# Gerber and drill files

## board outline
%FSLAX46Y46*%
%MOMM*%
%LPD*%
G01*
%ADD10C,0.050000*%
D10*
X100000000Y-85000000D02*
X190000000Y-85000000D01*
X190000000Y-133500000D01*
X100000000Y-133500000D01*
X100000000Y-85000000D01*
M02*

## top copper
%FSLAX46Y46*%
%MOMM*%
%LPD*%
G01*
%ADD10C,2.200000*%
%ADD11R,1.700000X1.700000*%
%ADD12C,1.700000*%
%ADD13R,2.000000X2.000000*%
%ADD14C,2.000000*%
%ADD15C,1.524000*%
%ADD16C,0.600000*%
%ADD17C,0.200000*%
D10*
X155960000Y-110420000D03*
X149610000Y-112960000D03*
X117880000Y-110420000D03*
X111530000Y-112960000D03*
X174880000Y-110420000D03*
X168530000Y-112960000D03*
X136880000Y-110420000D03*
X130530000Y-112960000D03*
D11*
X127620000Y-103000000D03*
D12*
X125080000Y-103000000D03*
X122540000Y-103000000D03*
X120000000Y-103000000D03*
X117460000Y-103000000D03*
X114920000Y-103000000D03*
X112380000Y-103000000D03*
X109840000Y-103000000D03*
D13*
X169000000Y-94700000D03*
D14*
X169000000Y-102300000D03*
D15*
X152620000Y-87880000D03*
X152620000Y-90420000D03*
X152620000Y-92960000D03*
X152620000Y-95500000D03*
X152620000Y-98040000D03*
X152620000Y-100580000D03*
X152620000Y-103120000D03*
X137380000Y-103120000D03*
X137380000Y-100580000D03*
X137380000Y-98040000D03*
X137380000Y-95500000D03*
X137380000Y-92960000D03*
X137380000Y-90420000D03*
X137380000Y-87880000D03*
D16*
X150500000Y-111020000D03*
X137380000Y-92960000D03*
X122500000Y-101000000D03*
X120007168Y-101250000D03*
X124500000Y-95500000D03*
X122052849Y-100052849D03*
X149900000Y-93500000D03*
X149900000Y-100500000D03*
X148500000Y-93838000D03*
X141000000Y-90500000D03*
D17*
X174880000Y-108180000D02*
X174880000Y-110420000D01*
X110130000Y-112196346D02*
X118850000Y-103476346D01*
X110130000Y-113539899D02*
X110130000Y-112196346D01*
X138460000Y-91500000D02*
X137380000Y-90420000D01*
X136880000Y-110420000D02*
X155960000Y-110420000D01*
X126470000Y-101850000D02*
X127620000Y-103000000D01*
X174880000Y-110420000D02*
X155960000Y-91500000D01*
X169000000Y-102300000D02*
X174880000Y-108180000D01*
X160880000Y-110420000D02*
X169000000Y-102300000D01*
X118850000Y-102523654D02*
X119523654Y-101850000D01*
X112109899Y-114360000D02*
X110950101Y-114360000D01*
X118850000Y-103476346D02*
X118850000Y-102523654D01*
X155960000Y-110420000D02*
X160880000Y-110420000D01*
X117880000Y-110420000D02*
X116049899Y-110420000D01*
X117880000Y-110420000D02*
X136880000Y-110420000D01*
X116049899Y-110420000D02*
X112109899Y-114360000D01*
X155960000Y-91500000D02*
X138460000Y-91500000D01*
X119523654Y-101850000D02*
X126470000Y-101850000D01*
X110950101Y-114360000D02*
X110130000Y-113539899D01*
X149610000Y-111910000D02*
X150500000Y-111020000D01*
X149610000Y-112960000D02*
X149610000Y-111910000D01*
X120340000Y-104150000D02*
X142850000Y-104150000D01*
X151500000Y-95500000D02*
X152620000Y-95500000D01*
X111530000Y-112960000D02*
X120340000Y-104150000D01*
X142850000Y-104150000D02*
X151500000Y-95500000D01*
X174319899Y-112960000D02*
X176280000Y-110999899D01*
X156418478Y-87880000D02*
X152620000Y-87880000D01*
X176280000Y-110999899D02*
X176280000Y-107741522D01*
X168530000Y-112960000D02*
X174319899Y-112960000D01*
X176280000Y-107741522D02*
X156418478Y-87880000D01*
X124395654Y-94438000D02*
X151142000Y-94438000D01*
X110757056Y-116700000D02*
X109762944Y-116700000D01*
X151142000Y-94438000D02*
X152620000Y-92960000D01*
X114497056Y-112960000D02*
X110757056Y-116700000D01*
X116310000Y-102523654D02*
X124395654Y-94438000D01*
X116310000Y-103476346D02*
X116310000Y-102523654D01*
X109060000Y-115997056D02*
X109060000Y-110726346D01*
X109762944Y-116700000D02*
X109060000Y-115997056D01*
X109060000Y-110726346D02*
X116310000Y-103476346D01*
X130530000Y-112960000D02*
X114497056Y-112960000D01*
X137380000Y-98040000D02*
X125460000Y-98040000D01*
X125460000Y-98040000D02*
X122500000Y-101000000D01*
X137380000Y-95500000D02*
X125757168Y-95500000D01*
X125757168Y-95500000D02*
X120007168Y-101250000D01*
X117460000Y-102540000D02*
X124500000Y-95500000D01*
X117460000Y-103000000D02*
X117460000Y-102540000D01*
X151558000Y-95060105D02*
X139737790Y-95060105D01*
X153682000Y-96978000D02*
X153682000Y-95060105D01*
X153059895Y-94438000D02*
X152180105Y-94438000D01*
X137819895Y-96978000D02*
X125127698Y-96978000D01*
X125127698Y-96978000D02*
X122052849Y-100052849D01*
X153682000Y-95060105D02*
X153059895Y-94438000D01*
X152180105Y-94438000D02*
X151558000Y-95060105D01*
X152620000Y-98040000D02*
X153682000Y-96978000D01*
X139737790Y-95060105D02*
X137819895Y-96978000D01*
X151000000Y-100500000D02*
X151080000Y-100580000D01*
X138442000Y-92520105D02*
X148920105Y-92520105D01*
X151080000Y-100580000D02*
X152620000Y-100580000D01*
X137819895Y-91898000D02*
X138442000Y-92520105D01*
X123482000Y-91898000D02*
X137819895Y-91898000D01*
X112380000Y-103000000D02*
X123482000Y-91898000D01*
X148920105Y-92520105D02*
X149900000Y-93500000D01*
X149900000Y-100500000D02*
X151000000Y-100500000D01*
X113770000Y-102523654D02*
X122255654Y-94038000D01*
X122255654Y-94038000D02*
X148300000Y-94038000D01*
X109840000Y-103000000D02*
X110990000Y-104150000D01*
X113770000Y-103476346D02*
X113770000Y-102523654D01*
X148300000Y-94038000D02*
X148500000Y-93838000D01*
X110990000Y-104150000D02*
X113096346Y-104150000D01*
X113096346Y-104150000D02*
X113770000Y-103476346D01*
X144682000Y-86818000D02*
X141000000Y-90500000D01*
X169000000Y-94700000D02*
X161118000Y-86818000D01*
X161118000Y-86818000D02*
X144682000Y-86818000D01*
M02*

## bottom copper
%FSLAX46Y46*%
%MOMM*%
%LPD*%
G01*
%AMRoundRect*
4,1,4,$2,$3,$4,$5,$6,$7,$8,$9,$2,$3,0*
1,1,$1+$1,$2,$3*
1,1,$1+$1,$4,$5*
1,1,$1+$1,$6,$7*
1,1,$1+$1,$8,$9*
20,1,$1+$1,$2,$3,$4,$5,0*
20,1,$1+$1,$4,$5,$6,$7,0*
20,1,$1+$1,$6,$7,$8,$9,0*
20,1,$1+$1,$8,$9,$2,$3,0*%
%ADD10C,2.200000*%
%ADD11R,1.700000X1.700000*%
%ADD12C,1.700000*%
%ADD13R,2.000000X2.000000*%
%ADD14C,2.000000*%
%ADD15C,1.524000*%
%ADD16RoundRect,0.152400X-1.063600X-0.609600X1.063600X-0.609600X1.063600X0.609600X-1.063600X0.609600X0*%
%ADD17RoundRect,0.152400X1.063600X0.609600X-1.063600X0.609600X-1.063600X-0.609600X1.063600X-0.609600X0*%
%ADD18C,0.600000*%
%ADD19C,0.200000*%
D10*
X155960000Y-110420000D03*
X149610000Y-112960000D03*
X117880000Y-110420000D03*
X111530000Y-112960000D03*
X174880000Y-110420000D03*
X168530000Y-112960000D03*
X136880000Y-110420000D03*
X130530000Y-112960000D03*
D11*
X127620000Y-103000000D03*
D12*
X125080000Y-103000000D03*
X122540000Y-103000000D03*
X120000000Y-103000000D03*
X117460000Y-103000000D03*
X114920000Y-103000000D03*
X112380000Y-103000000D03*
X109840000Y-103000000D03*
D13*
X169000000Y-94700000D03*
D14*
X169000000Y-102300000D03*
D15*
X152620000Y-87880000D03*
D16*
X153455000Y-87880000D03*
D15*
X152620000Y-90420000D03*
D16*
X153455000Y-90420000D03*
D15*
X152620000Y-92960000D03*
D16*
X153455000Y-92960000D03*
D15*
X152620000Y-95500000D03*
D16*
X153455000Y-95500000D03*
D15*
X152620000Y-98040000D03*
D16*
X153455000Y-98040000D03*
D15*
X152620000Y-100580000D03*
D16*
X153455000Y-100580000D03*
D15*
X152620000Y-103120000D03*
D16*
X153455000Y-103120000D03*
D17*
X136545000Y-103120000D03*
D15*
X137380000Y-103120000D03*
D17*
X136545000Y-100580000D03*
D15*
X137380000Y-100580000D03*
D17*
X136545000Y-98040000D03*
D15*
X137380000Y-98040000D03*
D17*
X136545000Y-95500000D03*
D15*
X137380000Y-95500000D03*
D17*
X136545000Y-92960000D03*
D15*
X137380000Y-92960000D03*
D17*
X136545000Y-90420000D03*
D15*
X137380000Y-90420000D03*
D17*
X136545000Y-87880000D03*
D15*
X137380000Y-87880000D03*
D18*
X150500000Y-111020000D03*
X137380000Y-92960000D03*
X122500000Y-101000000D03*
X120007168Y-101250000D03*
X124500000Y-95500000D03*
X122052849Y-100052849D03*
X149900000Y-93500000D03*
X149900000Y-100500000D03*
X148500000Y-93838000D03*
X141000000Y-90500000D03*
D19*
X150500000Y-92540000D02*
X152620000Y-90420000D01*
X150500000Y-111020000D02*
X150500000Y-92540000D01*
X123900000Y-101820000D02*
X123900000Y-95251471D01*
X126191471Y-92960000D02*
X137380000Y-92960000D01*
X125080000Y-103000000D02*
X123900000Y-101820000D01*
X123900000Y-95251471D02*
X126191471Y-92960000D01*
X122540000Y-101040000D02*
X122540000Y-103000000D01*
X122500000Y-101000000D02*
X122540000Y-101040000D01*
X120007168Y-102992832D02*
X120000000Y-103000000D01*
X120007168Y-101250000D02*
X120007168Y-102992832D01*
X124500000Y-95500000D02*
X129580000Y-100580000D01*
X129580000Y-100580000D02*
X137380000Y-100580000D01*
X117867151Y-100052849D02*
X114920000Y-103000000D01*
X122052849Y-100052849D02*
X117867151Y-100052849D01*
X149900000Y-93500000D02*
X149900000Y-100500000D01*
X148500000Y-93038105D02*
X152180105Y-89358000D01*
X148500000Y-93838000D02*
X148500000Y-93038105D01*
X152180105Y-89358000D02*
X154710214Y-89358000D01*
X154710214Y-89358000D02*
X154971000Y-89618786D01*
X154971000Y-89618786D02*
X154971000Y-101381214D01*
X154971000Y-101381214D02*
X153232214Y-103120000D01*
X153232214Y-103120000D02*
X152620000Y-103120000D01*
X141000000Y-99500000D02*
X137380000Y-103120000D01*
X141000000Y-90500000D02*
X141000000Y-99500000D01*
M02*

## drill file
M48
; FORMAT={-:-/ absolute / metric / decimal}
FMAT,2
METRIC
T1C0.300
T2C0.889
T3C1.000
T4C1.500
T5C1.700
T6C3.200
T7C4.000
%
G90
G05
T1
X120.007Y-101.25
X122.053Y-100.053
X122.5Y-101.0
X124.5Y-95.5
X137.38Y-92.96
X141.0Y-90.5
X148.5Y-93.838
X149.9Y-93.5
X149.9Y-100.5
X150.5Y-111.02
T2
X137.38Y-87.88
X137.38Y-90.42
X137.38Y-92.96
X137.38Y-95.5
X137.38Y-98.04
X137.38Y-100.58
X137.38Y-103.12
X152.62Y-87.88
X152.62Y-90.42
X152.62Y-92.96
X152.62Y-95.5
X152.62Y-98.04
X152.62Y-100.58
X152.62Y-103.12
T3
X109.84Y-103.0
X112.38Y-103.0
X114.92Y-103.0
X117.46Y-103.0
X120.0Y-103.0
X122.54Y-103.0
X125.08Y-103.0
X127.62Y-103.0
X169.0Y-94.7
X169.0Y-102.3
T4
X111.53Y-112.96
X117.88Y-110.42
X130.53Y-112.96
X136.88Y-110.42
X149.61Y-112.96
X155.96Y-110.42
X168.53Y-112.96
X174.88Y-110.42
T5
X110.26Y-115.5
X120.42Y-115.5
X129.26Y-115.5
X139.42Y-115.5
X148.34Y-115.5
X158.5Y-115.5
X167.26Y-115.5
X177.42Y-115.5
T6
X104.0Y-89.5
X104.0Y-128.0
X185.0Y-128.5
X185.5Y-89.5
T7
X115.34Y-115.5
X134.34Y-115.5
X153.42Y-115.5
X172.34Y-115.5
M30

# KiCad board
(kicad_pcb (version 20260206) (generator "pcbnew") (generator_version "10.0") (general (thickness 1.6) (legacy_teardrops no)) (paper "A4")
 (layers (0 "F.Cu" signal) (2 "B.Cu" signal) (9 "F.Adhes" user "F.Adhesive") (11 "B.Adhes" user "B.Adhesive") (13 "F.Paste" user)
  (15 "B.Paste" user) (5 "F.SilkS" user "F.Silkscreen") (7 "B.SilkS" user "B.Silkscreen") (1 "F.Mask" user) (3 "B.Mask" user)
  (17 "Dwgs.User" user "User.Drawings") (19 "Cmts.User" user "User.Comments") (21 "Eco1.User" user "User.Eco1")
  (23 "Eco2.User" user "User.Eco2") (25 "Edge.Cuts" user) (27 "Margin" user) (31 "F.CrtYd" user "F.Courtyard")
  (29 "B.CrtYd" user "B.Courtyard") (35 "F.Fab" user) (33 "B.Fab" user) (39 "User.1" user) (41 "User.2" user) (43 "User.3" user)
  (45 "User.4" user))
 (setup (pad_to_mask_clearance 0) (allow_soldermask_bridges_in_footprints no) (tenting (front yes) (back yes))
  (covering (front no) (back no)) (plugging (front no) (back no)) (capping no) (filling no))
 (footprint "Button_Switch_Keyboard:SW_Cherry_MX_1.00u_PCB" (layer "F.Cu") (at 155.96 110.42)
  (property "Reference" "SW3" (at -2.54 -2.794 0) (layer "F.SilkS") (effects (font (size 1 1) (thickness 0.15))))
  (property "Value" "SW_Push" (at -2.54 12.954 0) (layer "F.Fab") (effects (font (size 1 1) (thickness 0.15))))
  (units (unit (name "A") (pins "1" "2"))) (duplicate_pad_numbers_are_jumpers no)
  (pad "" np_thru_hole circle (at -7.62 5.08) (size 1.7 1.7) (drill 1.7) (layers "*.Cu" "*.Mask"))
  (pad "" np_thru_hole circle (at -2.54 5.08) (size 4 4) (drill 4) (layers "*.Cu" "*.Mask"))
  (pad "" np_thru_hole circle (at 2.54 5.08) (size 1.7 1.7) (drill 1.7) (layers "*.Cu" "*.Mask"))
  (pad "1" thru_hole circle (at 0 0) (size 2.2 2.2) (drill 1.5) (layers "*.Cu" "*.Mask") (remove_unused_layers no) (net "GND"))
  (pad "2" thru_hole circle (at -6.35 2.54) (size 2.2 2.2) (drill 1.5) (layers "*.Cu" "*.Mask") (remove_unused_layers no)
   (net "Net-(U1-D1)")))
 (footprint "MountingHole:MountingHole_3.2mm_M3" (layer "F.Cu") (at 104 89.5)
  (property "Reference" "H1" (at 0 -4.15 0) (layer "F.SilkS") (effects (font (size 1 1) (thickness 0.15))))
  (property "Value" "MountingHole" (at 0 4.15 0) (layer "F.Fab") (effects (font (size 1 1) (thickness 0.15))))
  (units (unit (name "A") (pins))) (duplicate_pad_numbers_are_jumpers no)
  (pad "" np_thru_hole circle (at 0 0) (size 3.2 3.2) (drill 3.2) (layers "*.Cu" "*.Mask")))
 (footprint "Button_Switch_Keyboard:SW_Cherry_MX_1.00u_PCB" (layer "F.Cu") (at 117.88 110.42)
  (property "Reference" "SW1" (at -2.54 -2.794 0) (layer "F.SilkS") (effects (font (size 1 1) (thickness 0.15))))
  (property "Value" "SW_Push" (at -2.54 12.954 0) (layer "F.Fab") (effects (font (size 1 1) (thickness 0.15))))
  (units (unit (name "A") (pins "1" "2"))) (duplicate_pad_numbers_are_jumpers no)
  (pad "" np_thru_hole circle (at -7.62 5.08) (size 1.7 1.7) (drill 1.7) (layers "*.Cu" "*.Mask"))
  (pad "" np_thru_hole circle (at -2.54 5.08) (size 4 4) (drill 4) (layers "*.Cu" "*.Mask"))
  (pad "" np_thru_hole circle (at 2.54 5.08) (size 1.7 1.7) (drill 1.7) (layers "*.Cu" "*.Mask"))
  (pad "1" thru_hole circle (at 0 0) (size 2.2 2.2) (drill 1.5) (layers "*.Cu" "*.Mask") (remove_unused_layers no) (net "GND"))
  (pad "2" thru_hole circle (at -6.35 2.54) (size 2.2 2.2) (drill 1.5) (layers "*.Cu" "*.Mask") (remove_unused_layers no)
   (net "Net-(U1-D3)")))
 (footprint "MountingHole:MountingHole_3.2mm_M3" (layer "F.Cu") (at 104 128)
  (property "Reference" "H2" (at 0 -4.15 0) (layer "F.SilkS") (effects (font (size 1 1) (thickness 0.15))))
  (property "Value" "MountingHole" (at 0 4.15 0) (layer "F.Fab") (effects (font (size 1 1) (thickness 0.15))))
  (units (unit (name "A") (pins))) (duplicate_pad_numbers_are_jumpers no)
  (pad "" np_thru_hole circle (at 0 0) (size 3.2 3.2) (drill 3.2) (layers "*.Cu" "*.Mask")))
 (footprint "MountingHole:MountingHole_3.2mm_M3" (layer "F.Cu") (at 185.5 89.5)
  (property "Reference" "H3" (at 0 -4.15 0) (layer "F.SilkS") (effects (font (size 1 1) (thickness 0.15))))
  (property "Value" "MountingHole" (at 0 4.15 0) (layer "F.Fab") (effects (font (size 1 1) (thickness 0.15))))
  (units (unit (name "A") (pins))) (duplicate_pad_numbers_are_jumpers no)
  (pad "" np_thru_hole circle (at 0 0) (size 3.2 3.2) (drill 3.2) (layers "*.Cu" "*.Mask")))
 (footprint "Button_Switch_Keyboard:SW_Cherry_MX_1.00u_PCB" (layer "F.Cu") (at 174.88 110.42)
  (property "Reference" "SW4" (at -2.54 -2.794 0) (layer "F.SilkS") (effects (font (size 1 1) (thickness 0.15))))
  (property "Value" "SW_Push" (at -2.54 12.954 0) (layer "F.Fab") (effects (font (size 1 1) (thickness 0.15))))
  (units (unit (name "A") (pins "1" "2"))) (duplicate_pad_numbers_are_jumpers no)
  (pad "" np_thru_hole circle (at -7.62 5.08) (size 1.7 1.7) (drill 1.7) (layers "*.Cu" "*.Mask"))
  (pad "" np_thru_hole circle (at -2.54 5.08) (size 4 4) (drill 4) (layers "*.Cu" "*.Mask"))
  (pad "" np_thru_hole circle (at 2.54 5.08) (size 1.7 1.7) (drill 1.7) (layers "*.Cu" "*.Mask"))
  (pad "1" thru_hole circle (at 0 0) (size 2.2 2.2) (drill 1.5) (layers "*.Cu" "*.Mask") (remove_unused_layers no) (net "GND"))
  (pad "2" thru_hole circle (at -6.35 2.54) (size 2.2 2.2) (drill 1.5) (layers "*.Cu" "*.Mask") (remove_unused_layers no)
   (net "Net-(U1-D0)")))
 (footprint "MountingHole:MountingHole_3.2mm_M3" (layer "F.Cu") (at 185 128.5)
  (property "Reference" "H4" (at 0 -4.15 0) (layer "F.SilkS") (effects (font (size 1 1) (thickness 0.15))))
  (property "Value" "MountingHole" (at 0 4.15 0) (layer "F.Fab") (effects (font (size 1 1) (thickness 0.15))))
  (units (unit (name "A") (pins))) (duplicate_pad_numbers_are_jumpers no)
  (pad "" np_thru_hole circle (at 0 0) (size 3.2 3.2) (drill 3.2) (layers "*.Cu" "*.Mask")))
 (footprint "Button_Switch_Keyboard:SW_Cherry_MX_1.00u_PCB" (layer "F.Cu") (at 136.88 110.42)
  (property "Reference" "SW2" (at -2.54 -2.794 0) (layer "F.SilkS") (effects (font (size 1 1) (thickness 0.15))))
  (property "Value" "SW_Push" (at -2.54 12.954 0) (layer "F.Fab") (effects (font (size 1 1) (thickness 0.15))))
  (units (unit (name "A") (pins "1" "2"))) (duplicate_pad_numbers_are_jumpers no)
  (pad "" np_thru_hole circle (at -7.62 5.08) (size 1.7 1.7) (drill 1.7) (layers "*.Cu" "*.Mask"))
  (pad "" np_thru_hole circle (at -2.54 5.08) (size 4 4) (drill 4) (layers "*.Cu" "*.Mask"))
  (pad "" np_thru_hole circle (at 2.54 5.08) (size 1.7 1.7) (drill 1.7) (layers "*.Cu" "*.Mask"))
  (pad "1" thru_hole circle (at 0 0) (size 2.2 2.2) (drill 1.5) (layers "*.Cu" "*.Mask") (remove_unused_layers no) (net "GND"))
  (pad "2" thru_hole circle (at -6.35 2.54) (size 2.2 2.2) (drill 1.5) (layers "*.Cu" "*.Mask") (remove_unused_layers no)
   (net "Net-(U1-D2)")))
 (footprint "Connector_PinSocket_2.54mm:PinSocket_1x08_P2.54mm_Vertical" (layer "B.Cu") (at 127.62 103 90)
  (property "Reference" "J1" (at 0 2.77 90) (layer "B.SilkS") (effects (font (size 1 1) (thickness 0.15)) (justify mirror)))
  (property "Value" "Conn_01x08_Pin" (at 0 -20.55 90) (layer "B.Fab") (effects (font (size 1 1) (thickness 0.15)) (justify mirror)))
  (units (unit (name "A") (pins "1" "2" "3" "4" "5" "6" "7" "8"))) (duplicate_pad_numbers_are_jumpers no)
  (pad "1" thru_hole rect (at 0 0 90) (size 1.7 1.7) (drill 1) (layers "*.Cu" "*.Mask") (remove_unused_layers no) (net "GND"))
  (pad "2" thru_hole circle (at 0 -2.54 90) (size 1.7 1.7) (drill 1) (layers "*.Cu" "*.Mask") (remove_unused_layers no) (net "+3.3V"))
  (pad "3" thru_hole circle (at 0 -5.08 90) (size 1.7 1.7) (drill 1) (layers "*.Cu" "*.Mask") (remove_unused_layers no) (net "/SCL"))
  (pad "4" thru_hole circle (at 0 -7.62 90) (size 1.7 1.7) (drill 1) (layers "*.Cu" "*.Mask") (remove_unused_layers no) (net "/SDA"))
  (pad "5" thru_hole circle (at 0 -10.16 90) (size 1.7 1.7) (drill 1) (layers "*.Cu" "*.Mask") (remove_unused_layers no) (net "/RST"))
  (pad "6" thru_hole circle (at 0 -12.7 90) (size 1.7 1.7) (drill 1) (layers "*.Cu" "*.Mask") (remove_unused_layers no) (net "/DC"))
  (pad "7" thru_hole circle (at 0 -15.24 90) (size 1.7 1.7) (drill 1) (layers "*.Cu" "*.Mask") (remove_unused_layers no) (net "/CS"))
  (pad "8" thru_hole circle (at 0 -17.78 90) (size 1.7 1.7) (drill 1) (layers "*.Cu" "*.Mask") (remove_unused_layers no) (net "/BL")))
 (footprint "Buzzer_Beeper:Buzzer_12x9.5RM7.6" (layer "B.Cu") (at 169 94.7 -90)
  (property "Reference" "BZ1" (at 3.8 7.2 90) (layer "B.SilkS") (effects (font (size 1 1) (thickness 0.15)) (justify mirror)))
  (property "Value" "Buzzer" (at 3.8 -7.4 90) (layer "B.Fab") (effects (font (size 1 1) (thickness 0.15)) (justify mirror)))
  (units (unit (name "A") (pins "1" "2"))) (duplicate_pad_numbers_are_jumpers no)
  (pad "1" thru_hole rect (at 0 0 270) (size 2 2) (drill 1) (layers "*.Cu" "*.Mask") (remove_unused_layers no) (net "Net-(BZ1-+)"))
  (pad "2" thru_hole circle (at 7.6 0 270) (size 2 2) (drill 1) (layers "*.Cu" "*.Mask") (remove_unused_layers no) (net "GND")))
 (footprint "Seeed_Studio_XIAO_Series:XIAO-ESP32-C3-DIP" (layer "B.Cu") (at 145 95.5 90)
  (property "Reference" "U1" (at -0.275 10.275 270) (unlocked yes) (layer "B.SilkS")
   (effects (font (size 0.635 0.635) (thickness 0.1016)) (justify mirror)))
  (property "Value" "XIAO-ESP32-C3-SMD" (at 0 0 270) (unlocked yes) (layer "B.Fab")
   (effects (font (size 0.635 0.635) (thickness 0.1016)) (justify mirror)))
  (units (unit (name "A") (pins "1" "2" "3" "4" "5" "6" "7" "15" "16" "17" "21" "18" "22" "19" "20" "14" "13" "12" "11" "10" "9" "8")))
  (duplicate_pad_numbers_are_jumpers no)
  (pad "1" thru_hole circle (at 7.62 7.62) (size 1.524 1.524) (drill 0.889) (layers "*.Cu" "*.Mask") (remove_unused_layers no)
   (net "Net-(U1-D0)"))
  (pad "1" smd roundrect (at 7.62 8.455) (size 2.432 1.524) (layers "B.Cu" "B.Mask") (roundrect_rratio 0.1) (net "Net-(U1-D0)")
   (thermal_bridge_angle 45))
  (pad "2" thru_hole circle (at 5.08 7.62) (size 1.524 1.524) (drill 0.889) (layers "*.Cu" "*.Mask") (remove_unused_layers no)
   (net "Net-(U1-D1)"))
  (pad "2" smd roundrect (at 5.08 8.455) (size 2.432 1.524) (layers "B.Cu" "B.Mask") (roundrect_rratio 0.1) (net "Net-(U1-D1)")
   (thermal_bridge_angle 45))
  (pad "3" thru_hole circle (at 2.54 7.62) (size 1.524 1.524) (drill 0.889) (layers "*.Cu" "*.Mask") (remove_unused_layers no)
   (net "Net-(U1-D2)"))
  (pad "3" smd roundrect (at 2.54 8.455) (size 2.432 1.524) (layers "B.Cu" "B.Mask") (roundrect_rratio 0.1) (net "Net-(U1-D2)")
   (thermal_bridge_angle 45))
  (pad "4" thru_hole circle (at 0 7.62) (size 1.524 1.524) (drill 0.889) (layers "*.Cu" "*.Mask") (remove_unused_layers no)
   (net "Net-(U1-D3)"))
  (pad "4" smd roundrect (at 0 8.455) (size 2.432 1.524) (layers "B.Cu" "B.Mask") (roundrect_rratio 0.1) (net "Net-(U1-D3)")
   (thermal_bridge_angle 45))
  (pad "5" thru_hole circle (at -2.54 7.62) (size 1.524 1.524) (drill 0.889) (layers "*.Cu" "*.Mask") (remove_unused_layers no) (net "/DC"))
  (pad "5" smd roundrect (at -2.54 8.455) (size 2.432 1.524) (layers "B.Cu" "B.Mask") (roundrect_rratio 0.1) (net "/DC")
   (thermal_bridge_angle 45))
  (pad "6" thru_hole circle (at -5.08 7.62) (size 1.524 1.524) (drill 0.889) (layers "*.Cu" "*.Mask") (remove_unused_layers no) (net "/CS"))
  (pad "6" smd roundrect (at -5.08 8.455) (size 2.432 1.524) (layers "B.Cu" "B.Mask") (roundrect_rratio 0.1) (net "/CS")
   (thermal_bridge_angle 45))
  (pad "7" thru_hole circle (at -7.62 7.62) (size 1.524 1.524) (drill 0.889) (layers "*.Cu" "*.Mask") (remove_unused_layers no) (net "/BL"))
  (pad "7" smd roundrect (at -7.62 8.455) (size 2.432 1.524) (layers "B.Cu" "B.Mask") (roundrect_rratio 0.1) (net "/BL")
   (thermal_bridge_angle 45))
  (pad "8" smd roundrect (at -7.62 -8.455 180) (size 2.432 1.524) (layers "B.Cu" "B.Mask") (roundrect_rratio 0.1) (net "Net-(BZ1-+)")
   (thermal_bridge_angle 45))
  (pad "8" thru_hole circle (at -7.62 -7.62 180) (size 1.524 1.524) (drill 0.889) (layers "*.Cu" "*.Mask") (remove_unused_layers no)
   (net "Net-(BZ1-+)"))
  (pad "9" smd roundrect (at -5.08 -8.455 180) (size 2.432 1.524) (layers "B.Cu" "B.Mask") (roundrect_rratio 0.1) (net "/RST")
   (thermal_bridge_angle 45))
  (pad "9" thru_hole circle (at -5.08 -7.62 180) (size 1.524 1.524) (drill 0.889) (layers "*.Cu" "*.Mask") (remove_unused_layers no)
   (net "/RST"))
  (pad "10" smd roundrect (at -2.54 -8.455 180) (size 2.432 1.524) (layers "B.Cu" "B.Mask") (roundrect_rratio 0.1) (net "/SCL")
   (thermal_bridge_angle 45))
  (pad "10" thru_hole circle (at -2.54 -7.62 180) (size 1.524 1.524) (drill 0.889) (layers "*.Cu" "*.Mask") (remove_unused_layers no)
   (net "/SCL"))
  (pad "11" smd roundrect (at 0 -8.455 180) (size 2.432 1.524) (layers "B.Cu" "B.Mask") (roundrect_rratio 0.1) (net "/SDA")
   (thermal_bridge_angle 45))
  (pad "11" thru_hole circle (at 0 -7.62 180) (size 1.524 1.524) (drill 0.889) (layers "*.Cu" "*.Mask") (remove_unused_layers no)
   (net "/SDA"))
  (pad "12" smd roundrect (at 2.54 -8.455 180) (size 2.432 1.524) (layers "B.Cu" "B.Mask") (roundrect_rratio 0.1) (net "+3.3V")
   (thermal_bridge_angle 45))
  (pad "12" thru_hole circle (at 2.54 -7.62 180) (size 1.524 1.524) (drill 0.889) (layers "*.Cu" "*.Mask") (remove_unused_layers no)
   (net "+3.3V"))
  (pad "13" smd roundrect (at 5.08 -8.455 180) (size 2.432 1.524) (layers "B.Cu" "B.Mask") (roundrect_rratio 0.1) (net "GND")
   (thermal_bridge_angle 45))
  (pad "13" thru_hole circle (at 5.08 -7.62 180) (size 1.524 1.524) (drill 0.889) (layers "*.Cu" "*.Mask") (remove_unused_layers no)
   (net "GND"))
  (pad "14" smd roundrect (at 7.62 -8.455 180) (size 2.432 1.524) (layers "B.Cu" "B.Mask") (roundrect_rratio 0.1)
   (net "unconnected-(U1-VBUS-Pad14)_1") (thermal_bridge_angle 45))
  (pad "14" thru_hole circle (at 7.62 -7.62 180) (size 1.524 1.524) (drill 0.889) (layers "*.Cu" "*.Mask") (remove_unused_layers no)
   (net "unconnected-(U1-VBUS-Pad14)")))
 (gr_rect (start 100 85) (end 190 133.5) (stroke (width 0.05) (type default)) (fill no) (layer "Edge.Cuts"))
 (segment (start 174.88 108.18) (end 174.88 110.42) (width 0.2) (layer "F.Cu") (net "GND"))
 (segment (start 110.13 112.196346) (end 118.85 103.476346) (width 0.2) (layer "F.Cu") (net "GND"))
 (segment (start 110.13 113.539899) (end 110.13 112.196346) (width 0.2) (layer "F.Cu") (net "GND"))
 (segment (start 138.46 91.5) (end 137.38 90.42) (width 0.2) (layer "F.Cu") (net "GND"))
 (segment (start 136.88 110.42) (end 155.96 110.42) (width 0.2) (layer "F.Cu") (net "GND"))
 (segment (start 126.47 101.85) (end 127.62 103) (width 0.2) (layer "F.Cu") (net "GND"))
 (segment (start 174.88 110.42) (end 155.96 91.5) (width 0.2) (layer "F.Cu") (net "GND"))
 (segment (start 169 102.3) (end 174.88 108.18) (width 0.2) (layer "F.Cu") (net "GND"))
 (segment (start 160.88 110.42) (end 169 102.3) (width 0.2) (layer "F.Cu") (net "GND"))
 (segment (start 118.85 102.523654) (end 119.523654 101.85) (width 0.2) (layer "F.Cu") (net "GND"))
 (segment (start 112.109899 114.36) (end 110.950101 114.36) (width 0.2) (layer "F.Cu") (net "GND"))
 (segment (start 118.85 103.476346) (end 118.85 102.523654) (width 0.2) (layer "F.Cu") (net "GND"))
 (segment (start 155.96 110.42) (end 160.88 110.42) (width 0.2) (layer "F.Cu") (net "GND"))
 (segment (start 117.88 110.42) (end 116.049899 110.42) (width 0.2) (layer "F.Cu") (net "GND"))
 (segment (start 117.88 110.42) (end 136.88 110.42) (width 0.2) (layer "F.Cu") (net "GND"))
 (segment (start 116.049899 110.42) (end 112.109899 114.36) (width 0.2) (layer "F.Cu") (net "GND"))
 (segment (start 155.96 91.5) (end 138.46 91.5) (width 0.2) (layer "F.Cu") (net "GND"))
 (segment (start 119.523654 101.85) (end 126.47 101.85) (width 0.2) (layer "F.Cu") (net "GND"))
 (segment (start 110.950101 114.36) (end 110.13 113.539899) (width 0.2) (layer "F.Cu") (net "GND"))
 (segment (start 149.61 111.91) (end 150.5 111.02) (width 0.2) (layer "F.Cu") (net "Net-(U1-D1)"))
 (segment (start 149.61 112.96) (end 149.61 111.91) (width 0.2) (layer "F.Cu") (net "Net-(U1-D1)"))
 (via (at 150.5 111.02) (size 0.6) (drill 0.3) (layers "F.Cu" "B.Cu") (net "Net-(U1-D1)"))
 (segment (start 150.5 92.54) (end 152.62 90.42) (width 0.2) (layer "B.Cu") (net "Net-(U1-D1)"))
 (segment (start 150.5 111.02) (end 150.5 92.54) (width 0.2) (layer "B.Cu") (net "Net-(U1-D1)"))
 (segment (start 120.34 104.15) (end 142.85 104.15) (width 0.2) (layer "F.Cu") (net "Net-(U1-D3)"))
 (segment (start 151.5 95.5) (end 152.62 95.5) (width 0.2) (layer "F.Cu") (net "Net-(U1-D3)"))
 (segment (start 111.53 112.96) (end 120.34 104.15) (width 0.2) (layer "F.Cu") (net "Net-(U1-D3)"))
 (segment (start 142.85 104.15) (end 151.5 95.5) (width 0.2) (layer "F.Cu") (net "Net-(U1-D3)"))
 (segment (start 174.319899 112.96) (end 176.28 110.999899) (width 0.2) (layer "F.Cu") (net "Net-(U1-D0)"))
 (segment (start 156.418478 87.88) (end 152.62 87.88) (width 0.2) (layer "F.Cu") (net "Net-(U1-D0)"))
 (segment (start 176.28 110.999899) (end 176.28 107.741522) (width 0.2) (layer "F.Cu") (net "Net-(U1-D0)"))
 (segment (start 168.53 112.96) (end 174.319899 112.96) (width 0.2) (layer "F.Cu") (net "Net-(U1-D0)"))
 (segment (start 176.28 107.741522) (end 156.418478 87.88) (width 0.2) (layer "F.Cu") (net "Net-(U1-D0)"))
 (segment (start 124.395654 94.438) (end 151.142 94.438) (width 0.2) (layer "F.Cu") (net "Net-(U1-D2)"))
 (segment (start 110.757056 116.7) (end 109.762944 116.7) (width 0.2) (layer "F.Cu") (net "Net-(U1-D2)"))
 (segment (start 151.142 94.438) (end 152.62 92.96) (width 0.2) (layer "F.Cu") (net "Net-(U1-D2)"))
 (segment (start 114.497056 112.96) (end 110.757056 116.7) (width 0.2) (layer "F.Cu") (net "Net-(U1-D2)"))
 (segment (start 116.31 102.523654) (end 124.395654 94.438) (width 0.2) (layer "F.Cu") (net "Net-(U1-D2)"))
 (segment (start 116.31 103.476346) (end 116.31 102.523654) (width 0.2) (layer "F.Cu") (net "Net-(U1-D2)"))
 (segment (start 109.06 115.997056) (end 109.06 110.726346) (width 0.2) (layer "F.Cu") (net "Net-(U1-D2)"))
 (segment (start 109.762944 116.7) (end 109.06 115.997056) (width 0.2) (layer "F.Cu") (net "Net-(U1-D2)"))
 (segment (start 109.06 110.726346) (end 116.31 103.476346) (width 0.2) (layer "F.Cu") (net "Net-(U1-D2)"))
 (segment (start 130.53 112.96) (end 114.497056 112.96) (width 0.2) (layer "F.Cu") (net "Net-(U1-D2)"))
 (via (at 137.38 92.96) (size 0.6) (drill 0.3) (layers "F.Cu" "B.Cu") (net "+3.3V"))
 (segment (start 123.9 101.82) (end 123.9 95.251471) (width 0.2) (layer "B.Cu") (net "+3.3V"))
 (segment (start 126.191471 92.96) (end 137.38 92.96) (width 0.2) (layer "B.Cu") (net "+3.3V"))
 (segment (start 125.08 103) (end 123.9 101.82) (width 0.2) (layer "B.Cu") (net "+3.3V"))
 (segment (start 123.9 95.251471) (end 126.191471 92.96) (width 0.2) (layer "B.Cu") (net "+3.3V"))
 (segment (start 137.38 98.04) (end 125.46 98.04) (width 0.2) (layer "F.Cu") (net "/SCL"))
 (segment (start 125.46 98.04) (end 122.5 101) (width 0.2) (layer "F.Cu") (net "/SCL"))
 (via (at 122.5 101) (size 0.6) (drill 0.3) (layers "F.Cu" "B.Cu") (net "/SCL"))
 (segment (start 122.54 101.04) (end 122.54 103) (width 0.2) (layer "B.Cu") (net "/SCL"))
 (segment (start 122.5 101) (end 122.54 101.04) (width 0.2) (layer "B.Cu") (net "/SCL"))
 (segment (start 137.38 95.5) (end 125.757168 95.5) (width 0.2) (layer "F.Cu") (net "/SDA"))
 (segment (start 125.757168 95.5) (end 120.007168 101.25) (width 0.2) (layer "F.Cu") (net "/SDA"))
 (via (at 120.007168 101.25) (size 0.6) (drill 0.3) (layers "F.Cu" "B.Cu") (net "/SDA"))
 (segment (start 120.007168 102.992832) (end 120 103) (width 0.2) (layer "B.Cu") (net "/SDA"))
 (segment (start 120.007168 101.25) (end 120.007168 102.992832) (width 0.2) (layer "B.Cu") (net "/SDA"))
 (segment (start 117.46 102.54) (end 124.5 95.5) (width 0.2) (layer "F.Cu") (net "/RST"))
 (segment (start 117.46 103) (end 117.46 102.54) (width 0.2) (layer "F.Cu") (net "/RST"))
 (via (at 124.5 95.5) (size 0.6) (drill 0.3) (layers "F.Cu" "B.Cu") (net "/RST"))
 (segment (start 124.5 95.5) (end 129.58 100.58) (width 0.2) (layer "B.Cu") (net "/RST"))
 (segment (start 129.58 100.58) (end 137.38 100.58) (width 0.2) (layer "B.Cu") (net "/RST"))
 (segment (start 151.558 95.060105) (end 139.73779 95.060105) (width 0.2) (layer "F.Cu") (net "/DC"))
 (segment (start 153.682 96.978) (end 153.682 95.060105) (width 0.2) (layer "F.Cu") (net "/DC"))
 (segment (start 153.059895 94.438) (end 152.180105 94.438) (width 0.2) (layer "F.Cu") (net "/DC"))
 (segment (start 137.819895 96.978) (end 125.127698 96.978) (width 0.2) (layer "F.Cu") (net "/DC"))
 (segment (start 125.127698 96.978) (end 122.052849 100.052849) (width 0.2) (layer "F.Cu") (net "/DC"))
 (segment (start 153.682 95.060105) (end 153.059895 94.438) (width 0.2) (layer "F.Cu") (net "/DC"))
 (segment (start 152.180105 94.438) (end 151.558 95.060105) (width 0.2) (layer "F.Cu") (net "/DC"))
 (segment (start 152.62 98.04) (end 153.682 96.978) (width 0.2) (layer "F.Cu") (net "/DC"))
 (segment (start 139.73779 95.060105) (end 137.819895 96.978) (width 0.2) (layer "F.Cu") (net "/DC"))
 (via (at 122.052849 100.052849) (size 0.6) (drill 0.3) (layers "F.Cu" "B.Cu") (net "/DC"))
 (segment (start 117.867151 100.052849) (end 114.92 103) (width 0.2) (layer "B.Cu") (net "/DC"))
 (segment (start 122.052849 100.052849) (end 117.867151 100.052849) (width 0.2) (layer "B.Cu") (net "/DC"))
 (segment (start 151 100.5) (end 151.08 100.58) (width 0.2) (layer "F.Cu") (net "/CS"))
 (segment (start 138.442 92.520105) (end 148.920105 92.520105) (width 0.2) (layer "F.Cu") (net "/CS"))
 (segment (start 151.08 100.58) (end 152.62 100.58) (width 0.2) (layer "F.Cu") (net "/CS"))
 (segment (start 137.819895 91.898) (end 138.442 92.520105) (width 0.2) (layer "F.Cu") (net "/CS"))
 (segment (start 123.482 91.898) (end 137.819895 91.898) (width 0.2) (layer "F.Cu") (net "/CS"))
 (segment (start 112.38 103) (end 123.482 91.898) (width 0.2) (layer "F.Cu") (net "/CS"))
 (segment (start 148.920105 92.520105) (end 149.9 93.5) (width 0.2) (layer "F.Cu") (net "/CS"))
 (segment (start 149.9 100.5) (end 151 100.5) (width 0.2) (layer "F.Cu") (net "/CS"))
 (via (at 149.9 93.5) (size 0.6) (drill 0.3) (layers "F.Cu" "B.Cu") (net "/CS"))
 (via (at 149.9 100.5) (size 0.6) (drill 0.3) (layers "F.Cu" "B.Cu") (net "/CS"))
 (segment (start 149.9 93.5) (end 149.9 100.5) (width 0.2) (layer "B.Cu") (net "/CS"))
 (segment (start 113.77 102.523654) (end 122.255654 94.038) (width 0.2) (layer "F.Cu") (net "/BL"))
 (segment (start 122.255654 94.038) (end 148.3 94.038) (width 0.2) (layer "F.Cu") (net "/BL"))
 (segment (start 109.84 103) (end 110.99 104.15) (width 0.2) (layer "F.Cu") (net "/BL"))
 (segment (start 113.77 103.476346) (end 113.77 102.523654) (width 0.2) (layer "F.Cu") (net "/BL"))
 (segment (start 148.3 94.038) (end 148.5 93.838) (width 0.2) (layer "F.Cu") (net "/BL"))
 (segment (start 110.99 104.15) (end 113.096346 104.15) (width 0.2) (layer "F.Cu") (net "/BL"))
 (segment (start 113.096346 104.15) (end 113.77 103.476346) (width 0.2) (layer "F.Cu") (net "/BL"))
 (via (at 148.5 93.838) (size 0.6) (drill 0.3) (layers "F.Cu" "B.Cu") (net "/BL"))
 (segment (start 148.5 93.038105) (end 152.180105 89.358) (width 0.2) (layer "B.Cu") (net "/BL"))
 (segment (start 148.5 93.838) (end 148.5 93.038105) (width 0.2) (layer "B.Cu") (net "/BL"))
 (segment (start 152.180105 89.358) (end 154.710214 89.358) (width 0.2) (layer "B.Cu") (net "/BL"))
 (segment (start 154.710214 89.358) (end 154.971 89.618786) (width 0.2) (layer "B.Cu") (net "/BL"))
 (segment (start 154.971 89.618786) (end 154.971 101.381214) (width 0.2) (layer "B.Cu") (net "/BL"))
 (segment (start 154.971 101.381214) (end 153.232214 103.12) (width 0.2) (layer "B.Cu") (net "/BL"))
 (segment (start 153.232214 103.12) (end 152.62 103.12) (width 0.2) (layer "B.Cu") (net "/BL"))
 (segment (start 144.682 86.818) (end 141 90.5) (width 0.2) (layer "F.Cu") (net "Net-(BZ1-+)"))
 (segment (start 169 94.7) (end 161.118 86.818) (width 0.2) (layer "F.Cu") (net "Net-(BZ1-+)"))
 (segment (start 161.118 86.818) (end 144.682 86.818) (width 0.2) (layer "F.Cu") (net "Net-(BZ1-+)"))
 (via (at 141 90.5) (size 0.6) (drill 0.3) (layers "F.Cu" "B.Cu") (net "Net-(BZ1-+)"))
 (segment (start 141 99.5) (end 137.38 103.12) (width 0.2) (layer "B.Cu") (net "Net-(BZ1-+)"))
 (segment (start 141 90.5) (end 141 99.5) (width 0.2) (layer "B.Cu") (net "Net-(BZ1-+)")))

